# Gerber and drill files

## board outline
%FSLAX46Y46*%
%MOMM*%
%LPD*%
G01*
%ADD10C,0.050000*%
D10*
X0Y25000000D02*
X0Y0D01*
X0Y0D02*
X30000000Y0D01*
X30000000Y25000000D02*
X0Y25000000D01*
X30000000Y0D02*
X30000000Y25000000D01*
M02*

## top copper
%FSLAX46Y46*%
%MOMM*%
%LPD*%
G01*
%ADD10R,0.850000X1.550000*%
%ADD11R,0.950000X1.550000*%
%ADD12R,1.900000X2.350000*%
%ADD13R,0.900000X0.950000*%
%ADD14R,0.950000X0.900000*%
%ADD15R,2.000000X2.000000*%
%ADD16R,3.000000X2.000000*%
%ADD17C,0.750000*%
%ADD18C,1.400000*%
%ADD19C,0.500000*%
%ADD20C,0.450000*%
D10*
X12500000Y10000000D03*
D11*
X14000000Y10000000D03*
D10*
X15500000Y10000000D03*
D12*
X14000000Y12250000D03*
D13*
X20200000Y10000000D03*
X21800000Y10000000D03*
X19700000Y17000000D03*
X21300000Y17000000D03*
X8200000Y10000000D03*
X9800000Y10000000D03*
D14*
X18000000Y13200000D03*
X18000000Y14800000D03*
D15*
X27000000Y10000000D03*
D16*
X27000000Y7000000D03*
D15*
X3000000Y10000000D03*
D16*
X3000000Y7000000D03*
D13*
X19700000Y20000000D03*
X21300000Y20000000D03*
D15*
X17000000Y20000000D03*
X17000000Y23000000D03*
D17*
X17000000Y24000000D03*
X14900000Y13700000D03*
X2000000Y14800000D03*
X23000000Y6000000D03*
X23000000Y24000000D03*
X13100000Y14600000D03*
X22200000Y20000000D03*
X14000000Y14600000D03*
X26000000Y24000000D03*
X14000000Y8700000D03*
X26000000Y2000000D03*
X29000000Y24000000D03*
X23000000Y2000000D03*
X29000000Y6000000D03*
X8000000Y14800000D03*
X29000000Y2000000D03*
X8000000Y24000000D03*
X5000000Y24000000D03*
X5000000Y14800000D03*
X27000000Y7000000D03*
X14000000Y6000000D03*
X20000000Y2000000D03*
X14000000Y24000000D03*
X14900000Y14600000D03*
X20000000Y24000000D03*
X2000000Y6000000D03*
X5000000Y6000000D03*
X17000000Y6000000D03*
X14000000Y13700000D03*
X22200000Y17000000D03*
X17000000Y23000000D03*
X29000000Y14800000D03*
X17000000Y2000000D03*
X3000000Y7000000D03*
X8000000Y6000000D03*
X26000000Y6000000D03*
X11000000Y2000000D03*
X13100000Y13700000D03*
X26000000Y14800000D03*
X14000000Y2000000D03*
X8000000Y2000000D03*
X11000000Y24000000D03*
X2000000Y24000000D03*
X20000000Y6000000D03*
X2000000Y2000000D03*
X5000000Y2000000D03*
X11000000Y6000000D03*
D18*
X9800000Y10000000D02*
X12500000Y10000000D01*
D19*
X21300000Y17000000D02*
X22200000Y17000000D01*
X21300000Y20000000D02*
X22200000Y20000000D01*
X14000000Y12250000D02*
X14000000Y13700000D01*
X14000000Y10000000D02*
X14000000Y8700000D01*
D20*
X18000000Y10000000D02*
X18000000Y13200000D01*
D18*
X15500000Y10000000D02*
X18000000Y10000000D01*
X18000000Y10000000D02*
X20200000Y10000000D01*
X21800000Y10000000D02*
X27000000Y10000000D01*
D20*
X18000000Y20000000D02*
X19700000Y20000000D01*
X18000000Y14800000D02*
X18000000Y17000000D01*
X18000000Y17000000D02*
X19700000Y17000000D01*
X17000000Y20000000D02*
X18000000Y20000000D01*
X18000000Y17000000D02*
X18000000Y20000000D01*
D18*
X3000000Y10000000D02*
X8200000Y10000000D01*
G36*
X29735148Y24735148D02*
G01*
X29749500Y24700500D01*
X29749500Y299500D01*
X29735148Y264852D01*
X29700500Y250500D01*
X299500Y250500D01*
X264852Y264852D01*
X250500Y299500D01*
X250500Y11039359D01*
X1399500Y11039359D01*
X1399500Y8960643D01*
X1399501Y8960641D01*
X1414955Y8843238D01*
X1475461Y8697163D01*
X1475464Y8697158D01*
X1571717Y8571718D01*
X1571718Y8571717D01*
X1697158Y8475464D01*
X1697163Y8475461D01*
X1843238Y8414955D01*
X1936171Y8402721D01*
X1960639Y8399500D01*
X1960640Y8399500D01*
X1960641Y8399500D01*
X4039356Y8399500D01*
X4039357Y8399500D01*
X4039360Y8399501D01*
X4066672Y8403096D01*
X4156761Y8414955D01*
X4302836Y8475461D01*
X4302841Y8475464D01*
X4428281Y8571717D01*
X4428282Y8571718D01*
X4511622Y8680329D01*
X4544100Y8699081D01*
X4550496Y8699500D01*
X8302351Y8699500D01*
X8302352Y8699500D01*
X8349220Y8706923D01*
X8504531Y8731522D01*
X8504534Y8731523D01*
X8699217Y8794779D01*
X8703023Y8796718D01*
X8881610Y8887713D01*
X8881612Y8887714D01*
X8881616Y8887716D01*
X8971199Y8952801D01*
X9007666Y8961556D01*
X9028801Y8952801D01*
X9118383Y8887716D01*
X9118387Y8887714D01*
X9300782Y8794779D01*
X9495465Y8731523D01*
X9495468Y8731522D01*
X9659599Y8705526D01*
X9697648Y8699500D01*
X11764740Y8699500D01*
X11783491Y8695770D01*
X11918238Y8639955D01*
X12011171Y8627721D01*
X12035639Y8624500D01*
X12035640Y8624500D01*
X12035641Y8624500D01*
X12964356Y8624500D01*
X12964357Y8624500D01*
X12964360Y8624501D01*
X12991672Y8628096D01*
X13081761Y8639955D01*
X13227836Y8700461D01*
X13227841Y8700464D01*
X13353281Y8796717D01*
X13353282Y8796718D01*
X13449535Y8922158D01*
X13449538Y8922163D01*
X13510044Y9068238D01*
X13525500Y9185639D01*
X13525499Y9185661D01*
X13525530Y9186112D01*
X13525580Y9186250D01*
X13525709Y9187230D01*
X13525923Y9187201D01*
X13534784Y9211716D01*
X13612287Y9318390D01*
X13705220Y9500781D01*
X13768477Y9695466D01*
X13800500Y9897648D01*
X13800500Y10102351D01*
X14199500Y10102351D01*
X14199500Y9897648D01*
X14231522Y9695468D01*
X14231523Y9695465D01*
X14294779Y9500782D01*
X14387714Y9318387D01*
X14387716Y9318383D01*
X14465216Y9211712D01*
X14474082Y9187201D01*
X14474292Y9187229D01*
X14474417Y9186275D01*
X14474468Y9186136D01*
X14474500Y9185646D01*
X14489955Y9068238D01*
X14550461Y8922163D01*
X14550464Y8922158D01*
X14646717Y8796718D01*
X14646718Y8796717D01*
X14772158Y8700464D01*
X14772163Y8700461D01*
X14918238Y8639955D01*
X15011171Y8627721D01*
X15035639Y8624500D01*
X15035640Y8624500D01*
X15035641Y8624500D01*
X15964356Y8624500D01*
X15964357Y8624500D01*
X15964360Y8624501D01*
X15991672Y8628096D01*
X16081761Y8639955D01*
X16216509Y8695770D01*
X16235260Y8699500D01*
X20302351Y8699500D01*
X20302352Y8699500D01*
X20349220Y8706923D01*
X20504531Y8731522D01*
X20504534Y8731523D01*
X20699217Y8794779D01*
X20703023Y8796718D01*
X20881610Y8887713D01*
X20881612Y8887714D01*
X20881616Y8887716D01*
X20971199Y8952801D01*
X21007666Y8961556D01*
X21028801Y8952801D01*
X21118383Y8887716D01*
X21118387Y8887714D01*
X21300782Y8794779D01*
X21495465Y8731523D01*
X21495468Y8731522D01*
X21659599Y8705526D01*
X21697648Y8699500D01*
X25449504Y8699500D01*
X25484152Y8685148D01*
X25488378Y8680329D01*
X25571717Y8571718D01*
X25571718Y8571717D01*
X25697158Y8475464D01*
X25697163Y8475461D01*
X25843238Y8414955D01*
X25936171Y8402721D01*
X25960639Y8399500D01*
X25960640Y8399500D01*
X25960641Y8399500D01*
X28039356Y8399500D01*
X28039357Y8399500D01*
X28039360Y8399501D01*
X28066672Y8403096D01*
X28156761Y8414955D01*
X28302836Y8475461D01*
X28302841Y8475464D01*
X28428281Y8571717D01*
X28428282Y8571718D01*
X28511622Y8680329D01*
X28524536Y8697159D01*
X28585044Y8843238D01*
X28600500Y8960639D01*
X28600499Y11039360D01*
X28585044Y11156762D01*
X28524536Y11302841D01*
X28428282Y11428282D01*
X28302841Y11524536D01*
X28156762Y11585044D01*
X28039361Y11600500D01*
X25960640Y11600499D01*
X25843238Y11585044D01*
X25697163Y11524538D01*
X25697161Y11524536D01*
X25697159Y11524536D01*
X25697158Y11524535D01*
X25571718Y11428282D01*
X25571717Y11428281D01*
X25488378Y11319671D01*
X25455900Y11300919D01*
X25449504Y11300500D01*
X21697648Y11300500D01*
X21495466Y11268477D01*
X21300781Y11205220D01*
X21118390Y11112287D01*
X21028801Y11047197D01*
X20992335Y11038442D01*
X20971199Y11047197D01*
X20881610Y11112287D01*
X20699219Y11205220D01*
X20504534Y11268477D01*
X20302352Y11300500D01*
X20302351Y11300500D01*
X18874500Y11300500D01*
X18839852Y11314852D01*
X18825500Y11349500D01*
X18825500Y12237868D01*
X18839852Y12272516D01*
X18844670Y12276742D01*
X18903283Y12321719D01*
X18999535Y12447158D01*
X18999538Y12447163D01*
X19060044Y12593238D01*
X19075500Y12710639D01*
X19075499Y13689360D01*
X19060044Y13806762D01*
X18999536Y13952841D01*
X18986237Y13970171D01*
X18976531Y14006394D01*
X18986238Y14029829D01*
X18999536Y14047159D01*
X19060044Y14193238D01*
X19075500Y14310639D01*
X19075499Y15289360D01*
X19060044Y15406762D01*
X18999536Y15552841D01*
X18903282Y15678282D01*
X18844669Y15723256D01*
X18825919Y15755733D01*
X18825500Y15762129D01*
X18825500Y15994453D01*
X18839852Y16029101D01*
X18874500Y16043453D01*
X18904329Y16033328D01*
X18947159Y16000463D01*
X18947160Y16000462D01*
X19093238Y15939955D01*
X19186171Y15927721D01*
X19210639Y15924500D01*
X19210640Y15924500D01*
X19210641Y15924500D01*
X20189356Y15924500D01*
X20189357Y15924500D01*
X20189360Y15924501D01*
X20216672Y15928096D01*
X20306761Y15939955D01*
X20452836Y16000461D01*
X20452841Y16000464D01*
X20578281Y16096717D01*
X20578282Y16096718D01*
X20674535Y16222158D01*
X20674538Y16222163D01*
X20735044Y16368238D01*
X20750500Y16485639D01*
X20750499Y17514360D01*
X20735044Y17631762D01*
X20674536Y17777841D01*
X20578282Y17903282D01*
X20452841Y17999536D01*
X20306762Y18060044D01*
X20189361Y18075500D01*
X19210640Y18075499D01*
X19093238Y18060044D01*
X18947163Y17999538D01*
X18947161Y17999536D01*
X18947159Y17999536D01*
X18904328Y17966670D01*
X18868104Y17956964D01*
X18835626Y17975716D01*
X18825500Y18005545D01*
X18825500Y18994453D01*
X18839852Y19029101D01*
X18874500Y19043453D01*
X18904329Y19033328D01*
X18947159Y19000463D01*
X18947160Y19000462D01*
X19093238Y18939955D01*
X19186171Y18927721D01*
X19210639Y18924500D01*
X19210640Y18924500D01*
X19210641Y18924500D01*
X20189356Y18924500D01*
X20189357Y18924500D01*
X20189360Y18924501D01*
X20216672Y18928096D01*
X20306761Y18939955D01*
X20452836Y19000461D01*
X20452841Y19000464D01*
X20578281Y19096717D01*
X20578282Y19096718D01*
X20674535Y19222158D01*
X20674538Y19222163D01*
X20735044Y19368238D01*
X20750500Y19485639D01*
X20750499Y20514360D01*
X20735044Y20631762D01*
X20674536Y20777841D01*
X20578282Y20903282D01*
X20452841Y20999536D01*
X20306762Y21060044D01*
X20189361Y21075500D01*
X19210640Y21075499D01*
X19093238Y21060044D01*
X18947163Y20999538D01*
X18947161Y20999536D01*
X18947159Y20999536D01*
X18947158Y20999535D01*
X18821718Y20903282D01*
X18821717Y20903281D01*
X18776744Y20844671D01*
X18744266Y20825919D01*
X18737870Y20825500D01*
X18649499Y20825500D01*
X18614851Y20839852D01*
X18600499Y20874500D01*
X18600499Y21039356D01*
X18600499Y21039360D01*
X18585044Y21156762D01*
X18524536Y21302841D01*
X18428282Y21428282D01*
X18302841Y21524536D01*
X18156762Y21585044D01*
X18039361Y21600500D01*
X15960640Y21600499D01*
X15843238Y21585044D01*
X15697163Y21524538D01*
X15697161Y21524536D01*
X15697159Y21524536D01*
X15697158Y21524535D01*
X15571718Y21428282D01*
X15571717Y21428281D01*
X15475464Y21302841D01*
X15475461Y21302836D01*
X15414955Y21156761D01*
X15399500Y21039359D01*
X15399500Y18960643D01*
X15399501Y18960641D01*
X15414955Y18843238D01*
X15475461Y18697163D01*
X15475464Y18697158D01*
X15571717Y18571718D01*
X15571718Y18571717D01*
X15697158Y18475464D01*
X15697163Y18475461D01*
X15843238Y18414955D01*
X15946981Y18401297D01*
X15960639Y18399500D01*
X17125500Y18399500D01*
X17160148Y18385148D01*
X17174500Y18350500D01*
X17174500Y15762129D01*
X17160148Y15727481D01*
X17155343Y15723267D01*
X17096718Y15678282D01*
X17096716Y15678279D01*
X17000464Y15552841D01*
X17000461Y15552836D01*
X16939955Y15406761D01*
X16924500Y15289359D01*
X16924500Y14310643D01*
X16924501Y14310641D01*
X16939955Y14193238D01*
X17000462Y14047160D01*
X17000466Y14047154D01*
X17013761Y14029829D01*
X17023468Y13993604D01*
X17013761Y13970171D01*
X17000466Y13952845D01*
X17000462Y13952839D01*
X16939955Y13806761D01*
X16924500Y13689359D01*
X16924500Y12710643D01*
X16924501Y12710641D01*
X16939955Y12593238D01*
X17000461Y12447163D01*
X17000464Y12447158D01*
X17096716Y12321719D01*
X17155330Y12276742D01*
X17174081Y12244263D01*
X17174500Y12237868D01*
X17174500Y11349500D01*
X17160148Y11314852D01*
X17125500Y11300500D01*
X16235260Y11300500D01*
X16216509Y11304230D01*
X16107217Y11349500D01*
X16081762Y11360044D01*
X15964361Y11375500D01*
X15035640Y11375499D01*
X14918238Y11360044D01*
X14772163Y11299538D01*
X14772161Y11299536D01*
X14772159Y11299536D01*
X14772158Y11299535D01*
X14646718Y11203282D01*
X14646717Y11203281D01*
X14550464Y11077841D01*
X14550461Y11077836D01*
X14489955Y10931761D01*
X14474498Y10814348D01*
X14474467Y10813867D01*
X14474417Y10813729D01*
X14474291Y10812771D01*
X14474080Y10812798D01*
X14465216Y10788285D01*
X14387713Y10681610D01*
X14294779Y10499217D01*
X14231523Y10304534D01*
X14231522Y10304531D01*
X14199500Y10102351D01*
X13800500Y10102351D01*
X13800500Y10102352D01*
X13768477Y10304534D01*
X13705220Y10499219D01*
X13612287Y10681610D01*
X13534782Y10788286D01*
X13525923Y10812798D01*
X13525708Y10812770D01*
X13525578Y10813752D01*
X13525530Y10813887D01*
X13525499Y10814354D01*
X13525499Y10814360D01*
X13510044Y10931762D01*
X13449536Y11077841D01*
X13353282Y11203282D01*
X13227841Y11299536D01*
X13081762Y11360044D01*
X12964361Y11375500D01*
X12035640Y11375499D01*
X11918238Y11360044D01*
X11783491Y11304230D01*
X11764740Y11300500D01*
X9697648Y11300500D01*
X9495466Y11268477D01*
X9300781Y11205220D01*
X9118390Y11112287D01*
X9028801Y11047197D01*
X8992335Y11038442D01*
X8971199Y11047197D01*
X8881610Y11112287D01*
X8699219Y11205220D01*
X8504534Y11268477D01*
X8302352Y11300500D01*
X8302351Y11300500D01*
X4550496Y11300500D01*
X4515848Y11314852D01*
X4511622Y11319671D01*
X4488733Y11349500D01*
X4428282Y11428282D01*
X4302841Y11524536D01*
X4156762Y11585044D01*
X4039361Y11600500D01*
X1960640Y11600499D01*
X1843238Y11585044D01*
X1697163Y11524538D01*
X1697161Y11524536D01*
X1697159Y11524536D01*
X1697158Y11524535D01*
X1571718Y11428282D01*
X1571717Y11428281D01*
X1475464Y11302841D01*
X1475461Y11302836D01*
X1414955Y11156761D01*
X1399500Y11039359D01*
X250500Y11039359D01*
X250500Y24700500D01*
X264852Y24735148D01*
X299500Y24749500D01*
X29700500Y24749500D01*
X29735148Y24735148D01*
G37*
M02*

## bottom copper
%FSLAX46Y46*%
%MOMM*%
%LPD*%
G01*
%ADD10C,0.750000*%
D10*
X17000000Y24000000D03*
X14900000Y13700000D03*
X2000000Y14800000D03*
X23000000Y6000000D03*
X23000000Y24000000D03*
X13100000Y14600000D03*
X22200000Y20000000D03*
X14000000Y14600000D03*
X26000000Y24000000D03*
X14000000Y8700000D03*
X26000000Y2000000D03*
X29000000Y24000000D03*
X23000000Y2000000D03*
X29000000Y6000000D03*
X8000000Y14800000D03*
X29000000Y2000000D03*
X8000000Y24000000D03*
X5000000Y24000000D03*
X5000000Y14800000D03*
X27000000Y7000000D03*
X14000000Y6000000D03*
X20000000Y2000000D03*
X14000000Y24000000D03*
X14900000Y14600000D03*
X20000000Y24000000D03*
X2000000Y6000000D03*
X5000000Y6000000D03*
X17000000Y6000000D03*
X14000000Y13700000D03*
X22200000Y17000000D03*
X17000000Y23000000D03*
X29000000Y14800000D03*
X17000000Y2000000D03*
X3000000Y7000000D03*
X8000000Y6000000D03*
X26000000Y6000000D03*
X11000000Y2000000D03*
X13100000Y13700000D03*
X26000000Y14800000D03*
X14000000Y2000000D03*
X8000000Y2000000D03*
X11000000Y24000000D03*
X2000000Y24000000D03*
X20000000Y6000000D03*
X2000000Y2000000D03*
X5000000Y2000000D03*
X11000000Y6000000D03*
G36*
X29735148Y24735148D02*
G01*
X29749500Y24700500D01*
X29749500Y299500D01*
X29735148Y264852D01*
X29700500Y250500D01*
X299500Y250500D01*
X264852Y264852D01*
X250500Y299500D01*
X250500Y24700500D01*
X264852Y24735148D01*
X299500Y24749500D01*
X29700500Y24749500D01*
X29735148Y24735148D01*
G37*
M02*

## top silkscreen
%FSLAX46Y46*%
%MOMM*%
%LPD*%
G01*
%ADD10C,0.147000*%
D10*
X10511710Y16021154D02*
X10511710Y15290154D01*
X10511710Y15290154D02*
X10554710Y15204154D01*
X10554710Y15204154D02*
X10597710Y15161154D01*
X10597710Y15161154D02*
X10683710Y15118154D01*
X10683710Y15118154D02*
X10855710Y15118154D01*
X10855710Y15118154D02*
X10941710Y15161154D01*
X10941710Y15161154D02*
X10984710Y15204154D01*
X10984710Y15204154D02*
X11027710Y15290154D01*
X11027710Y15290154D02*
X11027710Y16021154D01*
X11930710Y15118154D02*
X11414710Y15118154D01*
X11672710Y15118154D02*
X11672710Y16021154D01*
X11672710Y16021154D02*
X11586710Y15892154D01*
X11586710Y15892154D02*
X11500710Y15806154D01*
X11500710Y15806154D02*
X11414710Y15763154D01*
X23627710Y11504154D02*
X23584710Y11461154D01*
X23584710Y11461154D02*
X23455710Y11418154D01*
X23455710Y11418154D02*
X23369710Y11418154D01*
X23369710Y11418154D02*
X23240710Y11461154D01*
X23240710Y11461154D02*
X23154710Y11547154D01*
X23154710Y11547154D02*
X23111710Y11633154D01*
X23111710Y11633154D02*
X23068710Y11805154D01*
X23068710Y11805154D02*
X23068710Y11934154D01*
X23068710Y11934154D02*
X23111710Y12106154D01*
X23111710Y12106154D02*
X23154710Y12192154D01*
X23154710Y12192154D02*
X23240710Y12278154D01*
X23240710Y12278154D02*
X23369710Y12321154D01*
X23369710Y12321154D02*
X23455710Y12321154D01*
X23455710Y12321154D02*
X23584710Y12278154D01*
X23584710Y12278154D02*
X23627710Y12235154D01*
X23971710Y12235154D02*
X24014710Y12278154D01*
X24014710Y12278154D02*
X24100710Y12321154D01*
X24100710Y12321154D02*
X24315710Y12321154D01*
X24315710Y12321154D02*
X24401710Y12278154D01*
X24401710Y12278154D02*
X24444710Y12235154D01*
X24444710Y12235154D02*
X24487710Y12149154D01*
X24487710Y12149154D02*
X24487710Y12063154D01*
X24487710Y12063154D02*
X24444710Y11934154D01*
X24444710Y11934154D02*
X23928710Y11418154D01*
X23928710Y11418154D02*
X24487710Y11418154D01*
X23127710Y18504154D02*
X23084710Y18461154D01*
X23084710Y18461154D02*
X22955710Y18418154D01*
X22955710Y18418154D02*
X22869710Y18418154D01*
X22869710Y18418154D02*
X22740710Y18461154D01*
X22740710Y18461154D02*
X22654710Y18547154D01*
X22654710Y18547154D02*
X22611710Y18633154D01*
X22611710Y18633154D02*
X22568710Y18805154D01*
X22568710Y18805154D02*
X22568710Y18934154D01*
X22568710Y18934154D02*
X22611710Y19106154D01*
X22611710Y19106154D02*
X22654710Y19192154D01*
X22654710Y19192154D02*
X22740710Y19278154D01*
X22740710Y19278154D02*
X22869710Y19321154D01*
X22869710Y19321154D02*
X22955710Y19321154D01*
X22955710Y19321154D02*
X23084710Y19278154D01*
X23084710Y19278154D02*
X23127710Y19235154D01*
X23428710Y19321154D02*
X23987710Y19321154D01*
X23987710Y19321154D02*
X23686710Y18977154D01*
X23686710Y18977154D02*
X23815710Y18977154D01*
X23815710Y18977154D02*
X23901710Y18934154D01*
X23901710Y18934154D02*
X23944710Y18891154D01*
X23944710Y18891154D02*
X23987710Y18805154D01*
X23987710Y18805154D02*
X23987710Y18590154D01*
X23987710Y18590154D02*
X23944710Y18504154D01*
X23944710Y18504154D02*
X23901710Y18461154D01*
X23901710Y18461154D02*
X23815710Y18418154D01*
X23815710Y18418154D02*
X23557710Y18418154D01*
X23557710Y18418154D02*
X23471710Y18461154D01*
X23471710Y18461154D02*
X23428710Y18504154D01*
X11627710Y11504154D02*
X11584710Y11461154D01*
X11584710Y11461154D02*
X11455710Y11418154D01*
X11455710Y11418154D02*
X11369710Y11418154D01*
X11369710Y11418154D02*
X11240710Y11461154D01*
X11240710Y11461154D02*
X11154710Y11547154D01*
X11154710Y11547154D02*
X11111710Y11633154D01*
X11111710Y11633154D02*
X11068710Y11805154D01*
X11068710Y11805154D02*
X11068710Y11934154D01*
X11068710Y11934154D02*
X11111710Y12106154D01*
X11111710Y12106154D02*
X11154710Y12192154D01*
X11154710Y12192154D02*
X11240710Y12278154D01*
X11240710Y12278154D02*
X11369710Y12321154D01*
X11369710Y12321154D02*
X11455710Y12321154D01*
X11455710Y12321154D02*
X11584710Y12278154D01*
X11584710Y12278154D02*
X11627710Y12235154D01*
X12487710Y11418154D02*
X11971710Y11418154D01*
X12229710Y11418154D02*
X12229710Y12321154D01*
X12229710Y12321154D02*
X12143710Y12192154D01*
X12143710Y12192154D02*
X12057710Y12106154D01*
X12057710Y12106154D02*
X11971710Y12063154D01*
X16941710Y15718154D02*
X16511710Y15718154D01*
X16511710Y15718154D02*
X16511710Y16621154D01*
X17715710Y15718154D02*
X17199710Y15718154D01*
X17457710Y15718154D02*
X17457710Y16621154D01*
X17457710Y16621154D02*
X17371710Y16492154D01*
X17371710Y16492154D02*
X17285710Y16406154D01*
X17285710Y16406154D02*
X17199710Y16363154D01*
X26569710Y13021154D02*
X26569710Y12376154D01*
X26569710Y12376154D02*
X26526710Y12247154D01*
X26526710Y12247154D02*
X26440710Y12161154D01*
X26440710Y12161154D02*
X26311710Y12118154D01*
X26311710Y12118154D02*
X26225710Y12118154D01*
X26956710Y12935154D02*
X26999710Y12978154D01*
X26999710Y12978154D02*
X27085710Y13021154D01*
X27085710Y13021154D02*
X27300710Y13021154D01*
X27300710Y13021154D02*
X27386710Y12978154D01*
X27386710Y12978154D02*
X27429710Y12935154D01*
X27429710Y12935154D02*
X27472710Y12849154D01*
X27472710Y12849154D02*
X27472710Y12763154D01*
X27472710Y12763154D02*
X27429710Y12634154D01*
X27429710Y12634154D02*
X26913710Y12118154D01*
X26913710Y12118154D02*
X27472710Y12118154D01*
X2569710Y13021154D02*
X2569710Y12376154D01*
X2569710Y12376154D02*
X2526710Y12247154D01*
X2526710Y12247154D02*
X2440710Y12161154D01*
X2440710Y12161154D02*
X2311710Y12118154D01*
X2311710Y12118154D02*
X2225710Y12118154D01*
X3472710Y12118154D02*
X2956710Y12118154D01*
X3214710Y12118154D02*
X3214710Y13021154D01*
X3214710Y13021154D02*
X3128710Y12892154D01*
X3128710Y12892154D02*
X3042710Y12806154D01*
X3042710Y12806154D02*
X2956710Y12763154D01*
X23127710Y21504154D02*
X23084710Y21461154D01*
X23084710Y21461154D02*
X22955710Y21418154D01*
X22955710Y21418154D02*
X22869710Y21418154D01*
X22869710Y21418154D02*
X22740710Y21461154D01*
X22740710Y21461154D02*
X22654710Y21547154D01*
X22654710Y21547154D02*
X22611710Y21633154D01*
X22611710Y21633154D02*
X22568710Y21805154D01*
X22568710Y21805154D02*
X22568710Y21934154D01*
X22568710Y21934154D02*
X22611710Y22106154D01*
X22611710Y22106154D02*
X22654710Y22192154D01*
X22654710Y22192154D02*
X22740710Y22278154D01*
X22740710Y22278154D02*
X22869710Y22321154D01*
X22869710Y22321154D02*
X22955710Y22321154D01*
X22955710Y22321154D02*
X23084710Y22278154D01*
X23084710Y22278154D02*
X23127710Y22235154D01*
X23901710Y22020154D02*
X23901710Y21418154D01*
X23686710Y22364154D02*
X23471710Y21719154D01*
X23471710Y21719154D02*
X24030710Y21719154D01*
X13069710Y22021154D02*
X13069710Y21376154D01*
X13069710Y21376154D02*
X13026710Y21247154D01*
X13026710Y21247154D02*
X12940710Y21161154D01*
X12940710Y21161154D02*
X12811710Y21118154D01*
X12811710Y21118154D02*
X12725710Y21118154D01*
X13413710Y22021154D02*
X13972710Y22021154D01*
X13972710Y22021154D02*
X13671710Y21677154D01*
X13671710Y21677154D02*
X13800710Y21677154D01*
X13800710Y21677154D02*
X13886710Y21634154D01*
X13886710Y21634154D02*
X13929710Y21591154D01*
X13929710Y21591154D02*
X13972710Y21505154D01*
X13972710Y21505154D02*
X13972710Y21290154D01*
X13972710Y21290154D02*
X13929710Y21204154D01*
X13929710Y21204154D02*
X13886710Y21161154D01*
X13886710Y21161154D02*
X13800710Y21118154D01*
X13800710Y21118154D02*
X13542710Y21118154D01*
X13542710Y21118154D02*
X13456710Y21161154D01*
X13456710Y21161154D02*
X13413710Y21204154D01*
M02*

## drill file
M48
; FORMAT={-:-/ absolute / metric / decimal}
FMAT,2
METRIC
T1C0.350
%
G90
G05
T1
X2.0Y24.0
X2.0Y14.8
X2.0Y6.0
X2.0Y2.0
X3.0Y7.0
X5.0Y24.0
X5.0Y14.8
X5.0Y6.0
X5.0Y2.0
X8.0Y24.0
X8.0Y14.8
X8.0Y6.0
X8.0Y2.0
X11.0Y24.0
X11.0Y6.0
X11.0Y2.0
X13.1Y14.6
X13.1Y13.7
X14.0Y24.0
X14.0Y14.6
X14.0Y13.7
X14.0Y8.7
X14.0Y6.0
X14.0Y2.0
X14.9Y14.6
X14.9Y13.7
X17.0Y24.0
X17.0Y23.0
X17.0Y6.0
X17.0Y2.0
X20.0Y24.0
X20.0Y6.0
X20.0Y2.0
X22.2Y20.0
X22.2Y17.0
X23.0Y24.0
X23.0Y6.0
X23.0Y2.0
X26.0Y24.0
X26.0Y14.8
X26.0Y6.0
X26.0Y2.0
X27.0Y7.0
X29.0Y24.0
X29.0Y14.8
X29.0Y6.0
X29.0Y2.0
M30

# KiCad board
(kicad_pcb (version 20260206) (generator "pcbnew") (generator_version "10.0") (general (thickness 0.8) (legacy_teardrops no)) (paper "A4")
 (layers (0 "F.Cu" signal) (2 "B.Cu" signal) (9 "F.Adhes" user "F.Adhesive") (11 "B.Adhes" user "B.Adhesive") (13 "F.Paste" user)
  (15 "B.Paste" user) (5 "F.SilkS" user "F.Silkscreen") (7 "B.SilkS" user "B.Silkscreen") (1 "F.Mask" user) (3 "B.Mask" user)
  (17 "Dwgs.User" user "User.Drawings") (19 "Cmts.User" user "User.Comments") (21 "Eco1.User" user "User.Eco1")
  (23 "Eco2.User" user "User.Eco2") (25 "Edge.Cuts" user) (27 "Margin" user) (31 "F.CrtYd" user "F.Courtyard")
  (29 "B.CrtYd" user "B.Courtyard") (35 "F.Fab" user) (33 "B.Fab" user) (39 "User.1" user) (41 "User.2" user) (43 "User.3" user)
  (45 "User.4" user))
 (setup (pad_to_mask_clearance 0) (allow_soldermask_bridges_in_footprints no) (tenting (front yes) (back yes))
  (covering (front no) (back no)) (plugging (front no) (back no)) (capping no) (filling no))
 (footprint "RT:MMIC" (layer "F.Cu") (at 14 -11.6)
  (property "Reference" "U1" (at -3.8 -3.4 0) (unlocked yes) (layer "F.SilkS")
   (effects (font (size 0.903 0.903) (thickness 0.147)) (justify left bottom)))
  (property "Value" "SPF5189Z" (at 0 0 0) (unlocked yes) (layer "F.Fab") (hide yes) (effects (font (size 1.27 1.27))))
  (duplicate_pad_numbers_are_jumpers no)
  (pad "1" smd rect (at -1.5 1.6) (size 0.85 1.55) (layers "F.Cu" "F.Mask" "F.Paste") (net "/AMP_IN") (solder_mask_margin 0.1016)
   (solder_paste_margin 0) (thermal_bridge_angle 0))
  (pad "2" smd rect (at 0 1.6) (size 0.95 1.55) (layers "F.Cu" "F.Mask" "F.Paste") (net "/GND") (solder_mask_margin 0.1016)
   (solder_paste_margin 0) (thermal_bridge_angle 0))
  (pad "3" smd rect (at 1.5 1.6) (size 0.85 1.55) (layers "F.Cu" "F.Mask" "F.Paste") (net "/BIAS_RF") (solder_mask_margin 0.1016)
   (solder_paste_margin 0) (thermal_bridge_angle 0))
  (pad "4" smd rect (at 0 -0.65) (size 1.9 2.35) (layers "F.Cu" "F.Mask" "F.Paste") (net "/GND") (solder_mask_margin 0.1016)
   (solder_paste_margin 0) (thermal_bridge_angle 0)))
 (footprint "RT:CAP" (layer "F.Cu") (at 21 -10)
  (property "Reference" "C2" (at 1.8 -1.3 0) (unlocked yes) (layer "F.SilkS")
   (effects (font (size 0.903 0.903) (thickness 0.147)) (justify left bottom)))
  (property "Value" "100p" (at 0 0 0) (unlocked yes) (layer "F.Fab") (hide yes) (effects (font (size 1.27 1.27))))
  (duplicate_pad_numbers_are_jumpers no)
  (pad "1" smd rect (at -0.8 0) (size 0.9 0.95) (layers "F.Cu" "F.Mask" "F.Paste") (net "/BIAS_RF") (solder_mask_margin 0.1016)
   (solder_paste_margin 0) (thermal_bridge_angle 0))
  (pad "2" smd rect (at 0.8 0) (size 0.9 0.95) (layers "F.Cu" "F.Mask" "F.Paste") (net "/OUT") (solder_mask_margin 0.1016)
   (solder_paste_margin 0) (thermal_bridge_angle 0)))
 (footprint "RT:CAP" (layer "F.Cu") (at 20.5 -17)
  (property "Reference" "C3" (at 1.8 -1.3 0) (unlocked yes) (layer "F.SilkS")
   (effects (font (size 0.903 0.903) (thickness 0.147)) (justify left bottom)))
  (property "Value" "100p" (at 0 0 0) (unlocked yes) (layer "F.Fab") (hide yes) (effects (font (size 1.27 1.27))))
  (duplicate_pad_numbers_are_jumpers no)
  (pad "1" smd rect (at -0.8 0) (size 0.9 0.95) (layers "F.Cu" "F.Mask" "F.Paste") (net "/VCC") (solder_mask_margin 0.1016)
   (solder_paste_margin 0) (thermal_bridge_angle 0))
  (pad "2" smd rect (at 0.8 0) (size 0.9 0.95) (layers "F.Cu" "F.Mask" "F.Paste") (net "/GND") (solder_mask_margin 0.1016)
   (solder_paste_margin 0) (thermal_bridge_angle 0)))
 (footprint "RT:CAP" (layer "F.Cu") (at 9 -10)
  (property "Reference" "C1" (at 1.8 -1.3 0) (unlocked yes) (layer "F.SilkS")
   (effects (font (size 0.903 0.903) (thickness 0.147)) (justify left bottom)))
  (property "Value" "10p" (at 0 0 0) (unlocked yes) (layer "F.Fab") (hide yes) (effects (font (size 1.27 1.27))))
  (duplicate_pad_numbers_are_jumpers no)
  (pad "1" smd rect (at -0.8 0) (size 0.9 0.95) (layers "F.Cu" "F.Mask" "F.Paste") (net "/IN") (solder_mask_margin 0.1016)
   (solder_paste_margin 0) (thermal_bridge_angle 0))
  (pad "2" smd rect (at 0.8 0) (size 0.9 0.95) (layers "F.Cu" "F.Mask" "F.Paste") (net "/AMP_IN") (solder_mask_margin 0.1016)
   (solder_paste_margin 0) (thermal_bridge_angle 0)))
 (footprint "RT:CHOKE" (layer "F.Cu") (at 18 -14)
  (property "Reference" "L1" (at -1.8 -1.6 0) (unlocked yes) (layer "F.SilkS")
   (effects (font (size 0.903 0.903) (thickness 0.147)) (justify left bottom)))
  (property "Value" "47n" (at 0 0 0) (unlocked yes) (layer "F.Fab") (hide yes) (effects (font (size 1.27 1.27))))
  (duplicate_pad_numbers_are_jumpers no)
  (pad "1" smd rect (at 0 0.8) (size 0.95 0.9) (layers "F.Cu" "F.Mask" "F.Paste") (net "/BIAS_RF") (solder_mask_margin 0.1016)
   (solder_paste_margin 0) (thermal_bridge_angle 0))
  (pad "2" smd rect (at 0 -0.8) (size 0.95 0.9) (layers "F.Cu" "F.Mask" "F.Paste") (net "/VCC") (solder_mask_margin 0.1016)
   (solder_paste_margin 0) (thermal_bridge_angle 0)))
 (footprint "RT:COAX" (layer "F.Cu") (at 27 -10)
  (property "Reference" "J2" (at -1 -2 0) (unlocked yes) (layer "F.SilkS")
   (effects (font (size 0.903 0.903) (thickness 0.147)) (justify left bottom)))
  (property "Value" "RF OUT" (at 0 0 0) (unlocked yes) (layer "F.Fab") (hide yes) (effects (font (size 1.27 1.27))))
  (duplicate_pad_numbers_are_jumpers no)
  (pad "1" smd rect (at 0 0) (size 2 2) (layers "F.Cu" "F.Mask" "F.Paste") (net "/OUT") (solder_mask_margin 0.1016) (solder_paste_margin 0)
   (thermal_bridge_angle 0))
  (pad "2" smd rect (at 0 3) (size 3 2) (layers "F.Cu" "F.Mask" "F.Paste") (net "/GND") (solder_mask_margin 0.1016) (solder_paste_margin 0)
   (thermal_bridge_angle 0)))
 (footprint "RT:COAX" (layer "F.Cu") (at 3 -10)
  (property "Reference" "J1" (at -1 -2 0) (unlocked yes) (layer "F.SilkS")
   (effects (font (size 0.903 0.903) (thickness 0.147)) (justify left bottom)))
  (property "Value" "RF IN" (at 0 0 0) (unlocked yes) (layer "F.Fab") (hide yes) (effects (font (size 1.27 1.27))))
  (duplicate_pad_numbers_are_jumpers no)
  (pad "1" smd rect (at 0 0) (size 2 2) (layers "F.Cu" "F.Mask" "F.Paste") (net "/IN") (solder_mask_margin 0.1016) (solder_paste_margin 0)
   (thermal_bridge_angle 0))
  (pad "2" smd rect (at 0 3) (size 3 2) (layers "F.Cu" "F.Mask" "F.Paste") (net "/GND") (solder_mask_margin 0.1016) (solder_paste_margin 0)
   (thermal_bridge_angle 0)))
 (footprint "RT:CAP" (layer "F.Cu") (at 20.5 -20)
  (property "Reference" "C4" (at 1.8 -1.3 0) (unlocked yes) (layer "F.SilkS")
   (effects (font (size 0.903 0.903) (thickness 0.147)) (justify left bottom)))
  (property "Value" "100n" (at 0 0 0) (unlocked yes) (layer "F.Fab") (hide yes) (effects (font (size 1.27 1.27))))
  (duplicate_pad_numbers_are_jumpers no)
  (pad "1" smd rect (at -0.8 0) (size 0.9 0.95) (layers "F.Cu" "F.Mask" "F.Paste") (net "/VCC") (solder_mask_margin 0.1016)
   (solder_paste_margin 0) (thermal_bridge_angle 0))
  (pad "2" smd rect (at 0.8 0) (size 0.9 0.95) (layers "F.Cu" "F.Mask" "F.Paste") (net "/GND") (solder_mask_margin 0.1016)
   (solder_paste_margin 0) (thermal_bridge_angle 0)))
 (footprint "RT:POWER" (layer "F.Cu") (at 17 -20)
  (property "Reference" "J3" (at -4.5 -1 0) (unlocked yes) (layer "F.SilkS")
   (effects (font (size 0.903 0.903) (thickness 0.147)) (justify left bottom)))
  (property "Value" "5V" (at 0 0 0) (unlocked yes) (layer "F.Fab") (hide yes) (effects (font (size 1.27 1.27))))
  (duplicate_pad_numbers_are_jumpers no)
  (pad "1" smd rect (at 0 0) (size 2 2) (layers "F.Cu" "F.Mask" "F.Paste") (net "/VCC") (solder_mask_margin 0.1016) (solder_paste_margin 0)
   (thermal_bridge_angle 0))
  (pad "2" smd rect (at 0 -3) (size 2 2) (layers "F.Cu" "F.Mask" "F.Paste") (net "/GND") (solder_mask_margin 0.1016) (solder_paste_margin 0)
   (thermal_bridge_angle 0)))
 (gr_line (start 0 -25) (end 0 0) (stroke (width 0.05) (type solid)) (layer "Edge.Cuts"))
 (gr_line (start 0 0) (end 30 0) (stroke (width 0.05) (type solid)) (layer "Edge.Cuts"))
 (gr_line (start 30 -25) (end 0 -25) (stroke (width 0.05) (type solid)) (layer "Edge.Cuts"))
 (gr_line (start 30 0) (end 30 -25) (stroke (width 0.05) (type solid)) (layer "Edge.Cuts"))
 (segment (start 9.8 -10) (end 12.5 -10) (width 1.4) (layer "F.Cu") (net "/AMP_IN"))
 (segment (start 21.3 -17) (end 22.2 -17) (width 0.5) (layer "F.Cu") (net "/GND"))
 (segment (start 21.3 -20) (end 22.2 -20) (width 0.5) (layer "F.Cu") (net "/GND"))
 (segment (start 14 -12.25) (end 14 -13.7) (width 0.5) (layer "F.Cu") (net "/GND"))
 (segment (start 14 -10) (end 14 -8.7) (width 0.5) (layer "F.Cu") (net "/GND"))
 (via (at 17 -24) (size 0.75) (drill 0.35) (layers "F.Cu" "B.Cu") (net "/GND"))
 (via (at 14.9 -13.7) (size 0.75) (drill 0.35) (layers "F.Cu" "B.Cu") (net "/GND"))
 (via (at 2 -14.8) (size 0.75) (drill 0.35) (layers "F.Cu" "B.Cu") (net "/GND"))
 (via (at 23 -6) (size 0.75) (drill 0.35) (layers "F.Cu" "B.Cu") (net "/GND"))
 (via (at 23 -24) (size 0.75) (drill 0.35) (layers "F.Cu" "B.Cu") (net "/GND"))
 (via (at 13.1 -14.6) (size 0.75) (drill 0.35) (layers "F.Cu" "B.Cu") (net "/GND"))
 (via (at 22.2 -20) (size 0.75) (drill 0.35) (layers "F.Cu" "B.Cu") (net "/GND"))
 (via (at 14 -14.6) (size 0.75) (drill 0.35) (layers "F.Cu" "B.Cu") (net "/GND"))
 (via (at 26 -24) (size 0.75) (drill 0.35) (layers "F.Cu" "B.Cu") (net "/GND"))
 (via (at 14 -8.7) (size 0.75) (drill 0.35) (layers "F.Cu" "B.Cu") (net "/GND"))
 (via (at 26 -2) (size 0.75) (drill 0.35) (layers "F.Cu" "B.Cu") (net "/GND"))
 (via (at 29 -24) (size 0.75) (drill 0.35) (layers "F.Cu" "B.Cu") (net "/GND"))
 (via (at 23 -2) (size 0.75) (drill 0.35) (layers "F.Cu" "B.Cu") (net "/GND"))
 (via (at 29 -6) (size 0.75) (drill 0.35) (layers "F.Cu" "B.Cu") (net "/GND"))
 (via (at 8 -14.8) (size 0.75) (drill 0.35) (layers "F.Cu" "B.Cu") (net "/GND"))
 (via (at 29 -2) (size 0.75) (drill 0.35) (layers "F.Cu" "B.Cu") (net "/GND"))
 (via (at 8 -24) (size 0.75) (drill 0.35) (layers "F.Cu" "B.Cu") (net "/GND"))
 (via (at 5 -24) (size 0.75) (drill 0.35) (layers "F.Cu" "B.Cu") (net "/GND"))
 (via (at 5 -14.8) (size 0.75) (drill 0.35) (layers "F.Cu" "B.Cu") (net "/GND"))
 (via (at 27 -7) (size 0.75) (drill 0.35) (layers "F.Cu" "B.Cu") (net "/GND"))
 (via (at 14 -6) (size 0.75) (drill 0.35) (layers "F.Cu" "B.Cu") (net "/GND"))
 (via (at 20 -2) (size 0.75) (drill 0.35) (layers "F.Cu" "B.Cu") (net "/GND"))
 (via (at 14 -24) (size 0.75) (drill 0.35) (layers "F.Cu" "B.Cu") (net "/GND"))
 (via (at 14.9 -14.6) (size 0.75) (drill 0.35) (layers "F.Cu" "B.Cu") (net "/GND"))
 (via (at 20 -24) (size 0.75) (drill 0.35) (layers "F.Cu" "B.Cu") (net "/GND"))
 (via (at 2 -6) (size 0.75) (drill 0.35) (layers "F.Cu" "B.Cu") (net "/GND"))
 (via (at 5 -6) (size 0.75) (drill 0.35) (layers "F.Cu" "B.Cu") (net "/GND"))
 (via (at 17 -6) (size 0.75) (drill 0.35) (layers "F.Cu" "B.Cu") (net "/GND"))
 (via (at 14 -13.7) (size 0.75) (drill 0.35) (layers "F.Cu" "B.Cu") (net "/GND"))
 (via (at 22.2 -17) (size 0.75) (drill 0.35) (layers "F.Cu" "B.Cu") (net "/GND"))
 (via (at 17 -23) (size 0.75) (drill 0.35) (layers "F.Cu" "B.Cu") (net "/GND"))
 (via (at 29 -14.8) (size 0.75) (drill 0.35) (layers "F.Cu" "B.Cu") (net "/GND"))
 (via (at 17 -2) (size 0.75) (drill 0.35) (layers "F.Cu" "B.Cu") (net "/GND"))
 (via (at 3 -7) (size 0.75) (drill 0.35) (layers "F.Cu" "B.Cu") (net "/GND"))
 (via (at 8 -6) (size 0.75) (drill 0.35) (layers "F.Cu" "B.Cu") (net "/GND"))
 (via (at 26 -6) (size 0.75) (drill 0.35) (layers "F.Cu" "B.Cu") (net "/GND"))
 (via (at 11 -2) (size 0.75) (drill 0.35) (layers "F.Cu" "B.Cu") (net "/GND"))
 (via (at 13.1 -13.7) (size 0.75) (drill 0.35) (layers "F.Cu" "B.Cu") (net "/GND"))
 (via (at 26 -14.8) (size 0.75) (drill 0.35) (layers "F.Cu" "B.Cu") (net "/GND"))
 (via (at 14 -2) (size 0.75) (drill 0.35) (layers "F.Cu" "B.Cu") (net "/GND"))
 (via (at 8 -2) (size 0.75) (drill 0.35) (layers "F.Cu" "B.Cu") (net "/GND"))
 (via (at 11 -24) (size 0.75) (drill 0.35) (layers "F.Cu" "B.Cu") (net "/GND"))
 (via (at 2 -24) (size 0.75) (drill 0.35) (layers "F.Cu" "B.Cu") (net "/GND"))
 (via (at 20 -6) (size 0.75) (drill 0.35) (layers "F.Cu" "B.Cu") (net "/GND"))
 (via (at 2 -2) (size 0.75) (drill 0.35) (layers "F.Cu" "B.Cu") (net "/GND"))
 (via (at 5 -2) (size 0.75) (drill 0.35) (layers "F.Cu" "B.Cu") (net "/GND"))
 (via (at 11 -6) (size 0.75) (drill 0.35) (layers "F.Cu" "B.Cu") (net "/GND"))
 (segment (start 18 -10) (end 18 -13.2) (width 0.45) (layer "F.Cu") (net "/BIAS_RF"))
 (segment (start 15.5 -10) (end 18 -10) (width 1.4) (layer "F.Cu") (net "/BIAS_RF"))
 (segment (start 18 -10) (end 20.2 -10) (width 1.4) (layer "F.Cu") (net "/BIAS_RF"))
 (segment (start 21.8 -10) (end 27 -10) (width 1.4) (layer "F.Cu") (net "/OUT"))
 (segment (start 18 -20) (end 19.7 -20) (width 0.45) (layer "F.Cu") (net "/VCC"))
 (segment (start 18 -14.8) (end 18 -17) (width 0.45) (layer "F.Cu") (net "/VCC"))
 (segment (start 18 -17) (end 19.7 -17) (width 0.45) (layer "F.Cu") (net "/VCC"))
 (segment (start 17 -20) (end 18 -20) (width 0.45) (layer "F.Cu") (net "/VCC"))
 (segment (start 18 -17) (end 18 -20) (width 0.45) (layer "F.Cu") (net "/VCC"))
 (segment (start 3 -10) (end 8.2 -10) (width 1.4) (layer "F.Cu") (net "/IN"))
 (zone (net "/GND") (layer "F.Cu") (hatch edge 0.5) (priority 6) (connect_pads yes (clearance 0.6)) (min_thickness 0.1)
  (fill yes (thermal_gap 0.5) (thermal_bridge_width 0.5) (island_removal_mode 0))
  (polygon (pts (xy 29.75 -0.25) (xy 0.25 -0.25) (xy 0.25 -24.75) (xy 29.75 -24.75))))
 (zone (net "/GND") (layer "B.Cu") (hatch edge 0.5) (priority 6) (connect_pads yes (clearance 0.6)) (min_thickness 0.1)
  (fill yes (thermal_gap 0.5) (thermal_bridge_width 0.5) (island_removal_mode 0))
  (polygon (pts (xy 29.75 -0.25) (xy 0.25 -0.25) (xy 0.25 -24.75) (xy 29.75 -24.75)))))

